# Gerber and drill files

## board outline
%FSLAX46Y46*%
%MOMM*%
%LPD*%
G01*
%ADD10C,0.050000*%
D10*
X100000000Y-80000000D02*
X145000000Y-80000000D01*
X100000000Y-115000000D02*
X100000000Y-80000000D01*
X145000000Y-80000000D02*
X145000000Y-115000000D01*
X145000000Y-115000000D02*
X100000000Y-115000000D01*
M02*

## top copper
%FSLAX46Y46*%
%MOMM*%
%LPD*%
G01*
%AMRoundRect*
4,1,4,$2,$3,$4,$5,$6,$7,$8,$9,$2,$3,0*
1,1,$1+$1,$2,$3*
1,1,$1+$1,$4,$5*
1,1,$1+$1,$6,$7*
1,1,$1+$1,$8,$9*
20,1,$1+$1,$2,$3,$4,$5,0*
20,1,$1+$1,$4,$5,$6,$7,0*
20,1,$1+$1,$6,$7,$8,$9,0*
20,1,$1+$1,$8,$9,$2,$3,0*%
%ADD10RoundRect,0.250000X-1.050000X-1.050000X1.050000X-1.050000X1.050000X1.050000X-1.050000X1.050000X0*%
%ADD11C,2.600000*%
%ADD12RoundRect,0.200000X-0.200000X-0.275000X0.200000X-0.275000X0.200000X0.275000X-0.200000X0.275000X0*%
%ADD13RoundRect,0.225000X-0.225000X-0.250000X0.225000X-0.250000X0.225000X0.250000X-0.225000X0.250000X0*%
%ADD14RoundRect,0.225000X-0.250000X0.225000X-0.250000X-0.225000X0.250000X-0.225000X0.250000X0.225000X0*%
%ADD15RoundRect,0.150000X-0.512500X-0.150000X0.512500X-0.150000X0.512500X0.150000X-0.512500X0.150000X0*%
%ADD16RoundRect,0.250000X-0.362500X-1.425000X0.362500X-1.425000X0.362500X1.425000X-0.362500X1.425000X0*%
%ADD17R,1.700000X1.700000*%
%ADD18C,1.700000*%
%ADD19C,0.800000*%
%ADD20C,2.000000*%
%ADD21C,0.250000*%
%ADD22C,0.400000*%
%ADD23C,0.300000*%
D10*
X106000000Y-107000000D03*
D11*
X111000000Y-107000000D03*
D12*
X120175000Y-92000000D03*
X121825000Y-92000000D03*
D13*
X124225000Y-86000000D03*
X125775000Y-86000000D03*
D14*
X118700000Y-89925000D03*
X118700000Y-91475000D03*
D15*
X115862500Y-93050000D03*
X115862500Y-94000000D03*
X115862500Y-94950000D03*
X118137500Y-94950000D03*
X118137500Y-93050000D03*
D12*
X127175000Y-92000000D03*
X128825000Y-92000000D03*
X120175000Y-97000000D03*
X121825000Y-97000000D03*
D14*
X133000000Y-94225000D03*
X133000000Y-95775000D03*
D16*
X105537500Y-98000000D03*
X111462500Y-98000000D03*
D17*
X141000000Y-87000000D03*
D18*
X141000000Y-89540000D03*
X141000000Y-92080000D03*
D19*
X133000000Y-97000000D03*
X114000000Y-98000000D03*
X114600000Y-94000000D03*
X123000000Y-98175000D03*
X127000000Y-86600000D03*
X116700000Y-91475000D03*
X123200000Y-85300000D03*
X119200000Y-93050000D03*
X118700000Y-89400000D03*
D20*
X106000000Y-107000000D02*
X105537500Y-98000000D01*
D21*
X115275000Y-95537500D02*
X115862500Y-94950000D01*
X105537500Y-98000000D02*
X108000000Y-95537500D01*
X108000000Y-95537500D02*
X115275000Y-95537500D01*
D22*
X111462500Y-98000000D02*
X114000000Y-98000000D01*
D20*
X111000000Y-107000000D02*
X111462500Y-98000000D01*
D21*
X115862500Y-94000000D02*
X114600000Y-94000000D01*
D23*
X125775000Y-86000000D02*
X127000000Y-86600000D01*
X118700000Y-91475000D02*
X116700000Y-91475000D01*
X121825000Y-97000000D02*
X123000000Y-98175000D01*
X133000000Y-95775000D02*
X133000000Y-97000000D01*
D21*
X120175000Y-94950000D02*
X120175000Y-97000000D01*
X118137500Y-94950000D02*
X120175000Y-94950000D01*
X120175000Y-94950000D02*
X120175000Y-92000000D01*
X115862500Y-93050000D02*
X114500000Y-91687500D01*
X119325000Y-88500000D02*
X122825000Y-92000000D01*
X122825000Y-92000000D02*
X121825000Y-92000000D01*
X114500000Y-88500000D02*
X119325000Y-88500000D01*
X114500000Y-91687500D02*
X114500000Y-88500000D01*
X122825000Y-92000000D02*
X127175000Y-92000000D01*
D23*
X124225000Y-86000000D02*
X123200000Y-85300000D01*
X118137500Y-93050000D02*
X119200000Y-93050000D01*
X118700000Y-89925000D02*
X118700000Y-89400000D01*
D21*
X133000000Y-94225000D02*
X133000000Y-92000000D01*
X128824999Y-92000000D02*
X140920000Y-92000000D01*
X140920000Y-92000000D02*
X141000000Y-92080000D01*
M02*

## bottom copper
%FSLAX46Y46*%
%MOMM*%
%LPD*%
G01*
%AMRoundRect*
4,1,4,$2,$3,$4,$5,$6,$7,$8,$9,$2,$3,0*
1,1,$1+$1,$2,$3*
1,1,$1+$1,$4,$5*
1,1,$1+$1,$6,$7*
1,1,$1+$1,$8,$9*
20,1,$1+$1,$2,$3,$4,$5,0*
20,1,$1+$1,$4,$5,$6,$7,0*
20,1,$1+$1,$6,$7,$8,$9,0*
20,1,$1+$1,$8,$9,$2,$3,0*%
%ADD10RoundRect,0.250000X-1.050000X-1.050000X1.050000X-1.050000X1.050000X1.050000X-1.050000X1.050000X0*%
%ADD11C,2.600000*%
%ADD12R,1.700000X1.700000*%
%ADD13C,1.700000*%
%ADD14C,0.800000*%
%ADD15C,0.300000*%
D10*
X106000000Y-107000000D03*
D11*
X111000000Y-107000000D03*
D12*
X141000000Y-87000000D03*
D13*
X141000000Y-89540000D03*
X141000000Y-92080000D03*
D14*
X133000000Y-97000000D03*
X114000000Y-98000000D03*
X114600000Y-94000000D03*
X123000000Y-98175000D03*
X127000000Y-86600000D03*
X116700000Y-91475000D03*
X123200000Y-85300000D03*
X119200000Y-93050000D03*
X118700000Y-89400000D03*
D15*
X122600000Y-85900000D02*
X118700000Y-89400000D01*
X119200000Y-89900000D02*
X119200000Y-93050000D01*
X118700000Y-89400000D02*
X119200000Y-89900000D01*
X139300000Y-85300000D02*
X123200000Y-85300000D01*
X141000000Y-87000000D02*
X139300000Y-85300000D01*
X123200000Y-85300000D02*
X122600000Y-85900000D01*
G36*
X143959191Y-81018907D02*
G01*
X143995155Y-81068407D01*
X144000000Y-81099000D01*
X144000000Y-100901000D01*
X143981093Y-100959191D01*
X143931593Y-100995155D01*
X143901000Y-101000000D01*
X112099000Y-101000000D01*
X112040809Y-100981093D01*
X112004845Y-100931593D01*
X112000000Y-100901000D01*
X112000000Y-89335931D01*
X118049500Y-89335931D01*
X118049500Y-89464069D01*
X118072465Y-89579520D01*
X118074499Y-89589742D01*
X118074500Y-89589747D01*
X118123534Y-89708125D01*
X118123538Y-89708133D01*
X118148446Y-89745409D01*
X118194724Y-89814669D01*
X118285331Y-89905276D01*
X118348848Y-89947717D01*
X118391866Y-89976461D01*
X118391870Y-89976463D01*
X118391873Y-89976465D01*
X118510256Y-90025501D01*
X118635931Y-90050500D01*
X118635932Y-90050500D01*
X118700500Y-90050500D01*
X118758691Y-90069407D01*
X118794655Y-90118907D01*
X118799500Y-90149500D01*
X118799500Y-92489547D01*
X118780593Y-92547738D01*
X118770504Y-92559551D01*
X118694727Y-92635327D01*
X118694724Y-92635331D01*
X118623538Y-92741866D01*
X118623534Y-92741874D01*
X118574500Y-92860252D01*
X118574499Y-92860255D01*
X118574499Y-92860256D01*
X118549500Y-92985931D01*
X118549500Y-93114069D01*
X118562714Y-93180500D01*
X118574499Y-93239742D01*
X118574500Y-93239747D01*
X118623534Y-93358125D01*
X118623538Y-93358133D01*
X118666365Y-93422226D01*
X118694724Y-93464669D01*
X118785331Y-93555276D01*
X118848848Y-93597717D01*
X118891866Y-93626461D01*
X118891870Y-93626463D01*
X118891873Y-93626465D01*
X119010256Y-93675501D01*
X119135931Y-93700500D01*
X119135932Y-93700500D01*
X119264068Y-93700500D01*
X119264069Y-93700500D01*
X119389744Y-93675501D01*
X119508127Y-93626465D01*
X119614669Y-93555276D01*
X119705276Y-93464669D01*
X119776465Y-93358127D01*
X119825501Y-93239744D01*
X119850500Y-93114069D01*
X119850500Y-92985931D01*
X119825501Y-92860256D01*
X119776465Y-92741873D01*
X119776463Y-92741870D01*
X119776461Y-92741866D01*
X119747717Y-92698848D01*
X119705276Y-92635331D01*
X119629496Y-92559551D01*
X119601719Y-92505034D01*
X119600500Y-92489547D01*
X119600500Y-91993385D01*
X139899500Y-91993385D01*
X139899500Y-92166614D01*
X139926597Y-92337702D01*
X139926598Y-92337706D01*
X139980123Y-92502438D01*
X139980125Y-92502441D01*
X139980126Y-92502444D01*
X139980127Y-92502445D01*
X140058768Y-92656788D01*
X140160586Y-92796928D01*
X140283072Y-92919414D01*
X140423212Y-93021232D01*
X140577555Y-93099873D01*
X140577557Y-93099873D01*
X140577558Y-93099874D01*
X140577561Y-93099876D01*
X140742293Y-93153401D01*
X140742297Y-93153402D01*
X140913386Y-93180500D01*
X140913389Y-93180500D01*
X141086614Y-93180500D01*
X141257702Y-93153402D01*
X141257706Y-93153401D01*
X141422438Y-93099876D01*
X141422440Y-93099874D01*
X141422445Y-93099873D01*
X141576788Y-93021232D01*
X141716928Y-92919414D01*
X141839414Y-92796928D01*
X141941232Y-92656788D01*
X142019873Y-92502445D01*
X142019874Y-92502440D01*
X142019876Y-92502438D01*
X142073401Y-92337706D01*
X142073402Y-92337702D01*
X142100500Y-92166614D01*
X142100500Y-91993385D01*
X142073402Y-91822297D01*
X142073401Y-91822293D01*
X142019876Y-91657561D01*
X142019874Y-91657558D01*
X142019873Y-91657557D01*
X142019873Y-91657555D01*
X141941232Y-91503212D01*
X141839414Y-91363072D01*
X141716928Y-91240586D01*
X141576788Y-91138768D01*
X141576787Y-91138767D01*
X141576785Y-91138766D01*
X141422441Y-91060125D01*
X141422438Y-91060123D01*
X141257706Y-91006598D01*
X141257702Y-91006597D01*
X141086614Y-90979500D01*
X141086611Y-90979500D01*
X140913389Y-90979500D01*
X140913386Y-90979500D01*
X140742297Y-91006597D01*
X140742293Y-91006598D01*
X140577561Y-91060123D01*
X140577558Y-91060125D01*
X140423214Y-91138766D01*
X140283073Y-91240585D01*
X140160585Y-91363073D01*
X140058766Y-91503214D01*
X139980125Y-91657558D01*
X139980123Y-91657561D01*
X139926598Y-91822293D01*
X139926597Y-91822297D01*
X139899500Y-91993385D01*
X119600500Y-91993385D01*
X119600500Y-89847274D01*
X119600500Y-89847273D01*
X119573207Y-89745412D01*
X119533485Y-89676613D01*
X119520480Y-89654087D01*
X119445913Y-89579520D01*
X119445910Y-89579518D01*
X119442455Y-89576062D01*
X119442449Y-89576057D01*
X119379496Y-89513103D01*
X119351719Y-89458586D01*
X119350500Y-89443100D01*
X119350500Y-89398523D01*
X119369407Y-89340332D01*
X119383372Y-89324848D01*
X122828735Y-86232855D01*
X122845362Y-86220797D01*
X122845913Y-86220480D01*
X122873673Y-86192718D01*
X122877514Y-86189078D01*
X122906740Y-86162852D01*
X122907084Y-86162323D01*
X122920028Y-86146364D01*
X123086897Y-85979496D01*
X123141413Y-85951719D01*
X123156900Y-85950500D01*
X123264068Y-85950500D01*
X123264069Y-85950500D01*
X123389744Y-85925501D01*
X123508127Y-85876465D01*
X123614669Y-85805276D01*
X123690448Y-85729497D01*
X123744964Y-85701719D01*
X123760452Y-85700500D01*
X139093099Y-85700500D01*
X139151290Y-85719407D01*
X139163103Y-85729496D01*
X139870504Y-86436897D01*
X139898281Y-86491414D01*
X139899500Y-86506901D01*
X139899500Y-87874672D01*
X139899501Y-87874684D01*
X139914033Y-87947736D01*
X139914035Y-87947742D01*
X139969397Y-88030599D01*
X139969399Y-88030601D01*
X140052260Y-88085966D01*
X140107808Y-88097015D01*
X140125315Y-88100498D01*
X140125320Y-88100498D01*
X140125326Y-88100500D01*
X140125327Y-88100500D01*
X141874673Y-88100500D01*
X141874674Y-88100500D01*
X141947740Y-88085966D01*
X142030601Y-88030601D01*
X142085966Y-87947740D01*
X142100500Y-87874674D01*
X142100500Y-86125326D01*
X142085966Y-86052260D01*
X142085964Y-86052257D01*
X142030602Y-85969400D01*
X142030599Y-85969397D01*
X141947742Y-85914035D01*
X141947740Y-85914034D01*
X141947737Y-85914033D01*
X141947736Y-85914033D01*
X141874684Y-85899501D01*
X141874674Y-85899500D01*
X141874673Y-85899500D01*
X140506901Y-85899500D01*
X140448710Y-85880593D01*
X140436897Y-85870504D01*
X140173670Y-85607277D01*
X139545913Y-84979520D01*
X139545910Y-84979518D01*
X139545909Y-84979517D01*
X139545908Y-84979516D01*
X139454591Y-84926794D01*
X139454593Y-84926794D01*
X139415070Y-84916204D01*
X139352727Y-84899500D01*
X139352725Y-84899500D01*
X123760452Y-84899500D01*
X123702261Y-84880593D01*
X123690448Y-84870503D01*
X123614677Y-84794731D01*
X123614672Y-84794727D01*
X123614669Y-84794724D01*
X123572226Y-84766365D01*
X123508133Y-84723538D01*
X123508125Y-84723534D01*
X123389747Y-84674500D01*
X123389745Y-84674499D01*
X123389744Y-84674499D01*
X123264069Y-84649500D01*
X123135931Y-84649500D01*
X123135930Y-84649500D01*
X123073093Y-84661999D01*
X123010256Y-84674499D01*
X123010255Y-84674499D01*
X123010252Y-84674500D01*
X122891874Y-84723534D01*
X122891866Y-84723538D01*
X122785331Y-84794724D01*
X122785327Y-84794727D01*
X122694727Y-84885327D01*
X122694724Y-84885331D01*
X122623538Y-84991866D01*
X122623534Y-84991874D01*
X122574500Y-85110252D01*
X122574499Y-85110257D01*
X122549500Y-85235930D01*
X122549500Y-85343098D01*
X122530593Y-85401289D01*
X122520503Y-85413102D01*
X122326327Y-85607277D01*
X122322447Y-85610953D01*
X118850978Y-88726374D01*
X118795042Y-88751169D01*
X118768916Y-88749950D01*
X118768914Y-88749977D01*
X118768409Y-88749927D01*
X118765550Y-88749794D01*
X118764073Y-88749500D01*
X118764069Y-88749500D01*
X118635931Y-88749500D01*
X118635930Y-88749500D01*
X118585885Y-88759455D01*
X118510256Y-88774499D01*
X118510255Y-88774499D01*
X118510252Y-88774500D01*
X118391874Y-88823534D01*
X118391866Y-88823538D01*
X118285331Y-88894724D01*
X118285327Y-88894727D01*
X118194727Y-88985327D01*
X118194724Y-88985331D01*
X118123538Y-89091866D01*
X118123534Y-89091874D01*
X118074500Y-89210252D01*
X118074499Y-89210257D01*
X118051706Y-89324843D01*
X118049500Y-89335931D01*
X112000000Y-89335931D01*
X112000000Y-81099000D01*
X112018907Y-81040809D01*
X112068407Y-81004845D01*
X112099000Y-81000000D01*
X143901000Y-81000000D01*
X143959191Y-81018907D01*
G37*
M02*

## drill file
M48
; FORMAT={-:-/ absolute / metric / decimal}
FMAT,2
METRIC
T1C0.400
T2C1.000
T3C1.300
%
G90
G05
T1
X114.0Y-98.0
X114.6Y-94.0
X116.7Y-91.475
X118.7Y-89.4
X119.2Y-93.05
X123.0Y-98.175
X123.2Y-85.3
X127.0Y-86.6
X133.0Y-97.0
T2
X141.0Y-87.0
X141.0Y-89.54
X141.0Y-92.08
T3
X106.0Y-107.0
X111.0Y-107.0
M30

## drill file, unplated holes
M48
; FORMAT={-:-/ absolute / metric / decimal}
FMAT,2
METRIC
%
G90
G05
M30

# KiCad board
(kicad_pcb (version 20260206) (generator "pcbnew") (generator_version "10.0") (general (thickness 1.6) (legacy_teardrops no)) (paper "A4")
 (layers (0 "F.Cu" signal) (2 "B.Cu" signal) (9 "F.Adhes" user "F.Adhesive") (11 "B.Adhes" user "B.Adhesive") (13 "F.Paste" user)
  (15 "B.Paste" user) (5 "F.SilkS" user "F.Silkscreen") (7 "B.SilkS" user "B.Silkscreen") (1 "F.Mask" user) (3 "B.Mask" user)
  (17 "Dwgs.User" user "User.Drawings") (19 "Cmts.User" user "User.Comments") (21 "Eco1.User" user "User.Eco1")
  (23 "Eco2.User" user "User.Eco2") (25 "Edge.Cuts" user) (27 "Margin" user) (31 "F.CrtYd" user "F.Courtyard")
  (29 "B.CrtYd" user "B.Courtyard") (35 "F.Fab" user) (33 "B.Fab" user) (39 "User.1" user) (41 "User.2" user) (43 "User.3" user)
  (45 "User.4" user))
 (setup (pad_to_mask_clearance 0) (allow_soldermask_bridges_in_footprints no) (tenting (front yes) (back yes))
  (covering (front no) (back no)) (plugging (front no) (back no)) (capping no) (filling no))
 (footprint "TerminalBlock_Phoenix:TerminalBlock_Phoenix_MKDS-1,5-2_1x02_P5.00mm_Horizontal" (layer "F.Cu") (at 106 107)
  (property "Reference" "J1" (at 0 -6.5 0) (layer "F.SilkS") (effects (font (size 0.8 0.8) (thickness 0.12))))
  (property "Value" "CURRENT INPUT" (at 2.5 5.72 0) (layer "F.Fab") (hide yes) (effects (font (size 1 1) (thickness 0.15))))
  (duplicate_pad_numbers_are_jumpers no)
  (pad "1" thru_hole roundrect (at 0 0) (size 2.6 2.6) (drill 1.3) (layers "*.Cu" "*.Mask") (remove_unused_layers no)
   (roundrect_rratio 0.096154) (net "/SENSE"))
  (pad "2" thru_hole circle (at 5 0) (size 2.6 2.6) (drill 1.3) (layers "*.Cu" "*.Mask") (remove_unused_layers no) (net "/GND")))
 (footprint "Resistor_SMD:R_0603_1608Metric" (layer "F.Cu") (at 121 92)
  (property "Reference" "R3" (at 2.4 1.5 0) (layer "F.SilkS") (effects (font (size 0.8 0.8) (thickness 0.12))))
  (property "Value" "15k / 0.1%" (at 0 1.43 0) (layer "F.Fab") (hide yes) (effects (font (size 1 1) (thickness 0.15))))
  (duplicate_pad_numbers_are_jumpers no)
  (pad "1" smd roundrect (at -0.825 0) (size 0.8 0.95) (layers "F.Cu" "F.Mask" "F.Paste") (roundrect_rratio 0.25) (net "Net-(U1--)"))
  (pad "2" smd roundrect (at 0.825 0) (size 0.8 0.95) (layers "F.Cu" "F.Mask" "F.Paste") (roundrect_rratio 0.25) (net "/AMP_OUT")))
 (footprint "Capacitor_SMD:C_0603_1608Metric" (layer "F.Cu") (at 125 86)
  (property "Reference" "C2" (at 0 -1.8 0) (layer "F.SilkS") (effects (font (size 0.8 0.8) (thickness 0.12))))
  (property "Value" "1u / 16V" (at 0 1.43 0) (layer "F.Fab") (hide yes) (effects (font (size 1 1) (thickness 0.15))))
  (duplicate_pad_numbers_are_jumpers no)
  (pad "1" smd roundrect (at -0.775 0) (size 0.9 0.95) (layers "F.Cu" "F.Mask" "F.Paste") (roundrect_rratio 0.25) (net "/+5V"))
  (pad "2" smd roundrect (at 0.775 0) (size 0.9 0.95) (layers "F.Cu" "F.Mask" "F.Paste") (roundrect_rratio 0.25) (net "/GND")))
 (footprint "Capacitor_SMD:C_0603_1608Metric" (layer "F.Cu") (at 118.7 90.7 -90)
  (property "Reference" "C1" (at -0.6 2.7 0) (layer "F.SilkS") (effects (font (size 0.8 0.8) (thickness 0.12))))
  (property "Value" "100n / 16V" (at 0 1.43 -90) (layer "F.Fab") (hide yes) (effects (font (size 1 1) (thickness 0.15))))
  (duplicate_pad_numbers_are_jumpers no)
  (pad "1" smd roundrect (at -0.775 0 270) (size 0.9 0.95) (layers "F.Cu" "F.Mask" "F.Paste") (roundrect_rratio 0.25) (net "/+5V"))
  (pad "2" smd roundrect (at 0.775 0 270) (size 0.9 0.95) (layers "F.Cu" "F.Mask" "F.Paste") (roundrect_rratio 0.25) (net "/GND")))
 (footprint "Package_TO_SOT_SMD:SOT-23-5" (layer "F.Cu") (at 117 94)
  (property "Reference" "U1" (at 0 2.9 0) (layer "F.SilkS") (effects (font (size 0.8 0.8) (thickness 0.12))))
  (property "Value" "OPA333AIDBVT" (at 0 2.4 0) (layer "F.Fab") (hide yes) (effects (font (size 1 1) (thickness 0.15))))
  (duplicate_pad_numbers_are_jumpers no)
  (pad "1" smd roundrect (at -1.1375 -0.95) (size 1.325 0.6) (layers "F.Cu" "F.Mask" "F.Paste") (roundrect_rratio 0.25) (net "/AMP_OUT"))
  (pad "2" smd roundrect (at -1.1375 0) (size 1.325 0.6) (layers "F.Cu" "F.Mask" "F.Paste") (roundrect_rratio 0.25) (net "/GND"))
  (pad "3" smd roundrect (at -1.1375 0.95) (size 1.325 0.6) (layers "F.Cu" "F.Mask" "F.Paste") (roundrect_rratio 0.25) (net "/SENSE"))
  (pad "4" smd roundrect (at 1.1375 0.95) (size 1.325 0.6) (layers "F.Cu" "F.Mask" "F.Paste") (roundrect_rratio 0.25) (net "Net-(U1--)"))
  (pad "5" smd roundrect (at 1.1375 -0.95) (size 1.325 0.6) (layers "F.Cu" "F.Mask" "F.Paste") (roundrect_rratio 0.25) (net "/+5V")))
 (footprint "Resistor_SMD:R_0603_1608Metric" (layer "F.Cu") (at 128 92)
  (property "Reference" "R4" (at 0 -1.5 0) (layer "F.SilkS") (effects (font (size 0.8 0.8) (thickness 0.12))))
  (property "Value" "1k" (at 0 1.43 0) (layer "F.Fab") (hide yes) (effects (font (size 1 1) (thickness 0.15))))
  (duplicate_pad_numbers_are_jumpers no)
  (pad "1" smd roundrect (at -0.825 0) (size 0.8 0.95) (layers "F.Cu" "F.Mask" "F.Paste") (roundrect_rratio 0.25) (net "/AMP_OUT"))
  (pad "2" smd roundrect (at 0.825 0) (size 0.8 0.95) (layers "F.Cu" "F.Mask" "F.Paste") (roundrect_rratio 0.25) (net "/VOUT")))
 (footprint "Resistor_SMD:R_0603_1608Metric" (layer "F.Cu") (at 121 97)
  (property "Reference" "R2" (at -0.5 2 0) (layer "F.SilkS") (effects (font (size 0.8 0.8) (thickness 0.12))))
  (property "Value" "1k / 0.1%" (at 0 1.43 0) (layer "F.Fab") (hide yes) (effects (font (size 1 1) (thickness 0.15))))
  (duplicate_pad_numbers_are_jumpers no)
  (pad "1" smd roundrect (at -0.825 0) (size 0.8 0.95) (layers "F.Cu" "F.Mask" "F.Paste") (roundrect_rratio 0.25) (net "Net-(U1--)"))
  (pad "2" smd roundrect (at 0.825 0) (size 0.8 0.95) (layers "F.Cu" "F.Mask" "F.Paste") (roundrect_rratio 0.25) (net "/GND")))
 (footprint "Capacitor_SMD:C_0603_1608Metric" (layer "F.Cu") (at 133 95 -90)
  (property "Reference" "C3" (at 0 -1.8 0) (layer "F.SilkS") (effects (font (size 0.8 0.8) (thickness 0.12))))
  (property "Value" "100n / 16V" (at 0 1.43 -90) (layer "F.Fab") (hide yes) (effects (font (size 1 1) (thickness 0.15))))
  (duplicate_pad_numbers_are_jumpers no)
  (pad "1" smd roundrect (at -0.775 0 270) (size 0.9 0.95) (layers "F.Cu" "F.Mask" "F.Paste") (roundrect_rratio 0.25) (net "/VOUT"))
  (pad "2" smd roundrect (at 0.775 0 270) (size 0.9 0.95) (layers "F.Cu" "F.Mask" "F.Paste") (roundrect_rratio 0.25) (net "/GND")))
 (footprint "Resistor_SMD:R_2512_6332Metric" (layer "F.Cu") (at 108.5 98)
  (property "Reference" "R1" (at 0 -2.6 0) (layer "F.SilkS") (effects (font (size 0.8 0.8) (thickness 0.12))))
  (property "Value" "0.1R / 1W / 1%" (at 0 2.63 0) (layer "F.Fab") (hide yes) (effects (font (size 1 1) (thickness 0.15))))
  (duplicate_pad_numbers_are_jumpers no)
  (pad "1" smd roundrect (at -2.9625 0) (size 1.225 3.35) (layers "F.Cu" "F.Mask" "F.Paste") (roundrect_rratio 0.204082) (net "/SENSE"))
  (pad "2" smd roundrect (at 2.9625 0) (size 1.225 3.35) (layers "F.Cu" "F.Mask" "F.Paste") (roundrect_rratio 0.204082) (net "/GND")))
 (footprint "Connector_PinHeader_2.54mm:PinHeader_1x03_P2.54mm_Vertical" (layer "F.Cu") (at 141 87)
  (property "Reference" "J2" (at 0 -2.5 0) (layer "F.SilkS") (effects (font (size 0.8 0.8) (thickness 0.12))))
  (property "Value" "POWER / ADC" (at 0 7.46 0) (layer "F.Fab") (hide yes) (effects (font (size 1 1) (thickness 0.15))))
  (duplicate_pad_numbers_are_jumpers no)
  (pad "1" thru_hole rect (at 0 0) (size 1.7 1.7) (drill 1) (layers "*.Cu" "*.Mask") (remove_unused_layers no) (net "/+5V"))
  (pad "2" thru_hole circle (at 0 2.54) (size 1.7 1.7) (drill 1) (layers "*.Cu" "*.Mask") (remove_unused_layers no) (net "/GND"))
  (pad "3" thru_hole circle (at 0 5.08) (size 1.7 1.7) (drill 1) (layers "*.Cu" "*.Mask") (remove_unused_layers no) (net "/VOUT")))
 (gr_line (start 100 80) (end 145 80) (stroke (width 0.05) (type default)) (layer "Edge.Cuts"))
 (gr_line (start 100 115) (end 100 80) (stroke (width 0.05) (type default)) (layer "Edge.Cuts"))
 (gr_line (start 145 80) (end 145 115) (stroke (width 0.05) (type default)) (layer "Edge.Cuts"))
 (gr_line (start 145 115) (end 100 115) (stroke (width 0.05) (type default)) (layer "Edge.Cuts"))
 (segment (start 106 107) (end 105.5375 98) (width 2) (layer "F.Cu") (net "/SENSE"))
 (segment (start 115.275 95.5375) (end 115.8625 94.95) (width 0.25) (layer "F.Cu") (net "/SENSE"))
 (segment (start 105.5375 98) (end 108 95.5375) (width 0.25) (layer "F.Cu") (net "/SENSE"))
 (segment (start 108 95.5375) (end 115.275 95.5375) (width 0.25) (layer "F.Cu") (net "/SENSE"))
 (segment (start 111.4625 98) (end 114 98) (width 0.4) (layer "F.Cu") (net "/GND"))
 (segment (start 111 107) (end 111.4625 98) (width 2) (layer "F.Cu") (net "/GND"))
 (segment (start 115.8625 94) (end 114.6 94) (width 0.25) (layer "F.Cu") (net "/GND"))
 (segment (start 125.775 86) (end 127 86.6) (width 0.3) (layer "F.Cu") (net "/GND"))
 (segment (start 118.7 91.475) (end 116.7 91.475) (width 0.3) (layer "F.Cu") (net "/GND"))
 (segment (start 121.825 97) (end 123 98.175) (width 0.3) (layer "F.Cu") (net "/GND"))
 (segment (start 133 95.775) (end 133 97) (width 0.3) (layer "F.Cu") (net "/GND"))
 (via (at 133 97) (size 0.8) (drill 0.4) (layers "F.Cu" "B.Cu") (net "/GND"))
 (via (at 114 98) (size 0.8) (drill 0.4) (layers "F.Cu" "B.Cu") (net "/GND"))
 (via (at 114.6 94) (size 0.8) (drill 0.4) (layers "F.Cu" "B.Cu") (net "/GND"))
 (via (at 123 98.175) (size 0.8) (drill 0.4) (layers "F.Cu" "B.Cu") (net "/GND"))
 (via (at 127 86.6) (size 0.8) (drill 0.4) (layers "F.Cu" "B.Cu") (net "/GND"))
 (via (at 116.7 91.475) (size 0.8) (drill 0.4) (layers "F.Cu" "B.Cu") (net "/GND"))
 (segment (start 120.175 94.95) (end 120.175 97) (width 0.25) (layer "F.Cu") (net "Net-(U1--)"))
 (segment (start 118.1375 94.95) (end 120.175 94.95) (width 0.25) (layer "F.Cu") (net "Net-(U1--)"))
 (segment (start 120.175 94.95) (end 120.175 92) (width 0.25) (layer "F.Cu") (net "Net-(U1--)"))
 (segment (start 115.8625 93.05) (end 114.5 91.6875) (width 0.25) (layer "F.Cu") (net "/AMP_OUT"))
 (segment (start 119.325 88.5) (end 122.825 92) (width 0.25) (layer "F.Cu") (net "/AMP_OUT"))
 (segment (start 122.825 92) (end 121.825 92) (width 0.25) (layer "F.Cu") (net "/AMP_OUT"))
 (segment (start 114.5 88.5) (end 119.325 88.5) (width 0.25) (layer "F.Cu") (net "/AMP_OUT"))
 (segment (start 114.5 91.6875) (end 114.5 88.5) (width 0.25) (layer "F.Cu") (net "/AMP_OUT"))
 (segment (start 122.825 92) (end 127.175 92) (width 0.25) (layer "F.Cu") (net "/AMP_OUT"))
 (segment (start 124.225 86) (end 123.2 85.3) (width 0.3) (layer "F.Cu") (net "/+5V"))
 (segment (start 118.1375 93.05) (end 119.2 93.05) (width 0.3) (layer "F.Cu") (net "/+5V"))
 (segment (start 118.7 89.925) (end 118.7 89.4) (width 0.3) (layer "F.Cu") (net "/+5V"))
 (via (at 123.2 85.3) (size 0.8) (drill 0.4) (layers "F.Cu" "B.Cu") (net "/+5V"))
 (via (at 119.2 93.05) (size 0.8) (drill 0.4) (layers "F.Cu" "B.Cu") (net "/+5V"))
 (via (at 118.7 89.4) (size 0.8) (drill 0.4) (layers "F.Cu" "B.Cu") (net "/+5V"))
 (segment (start 122.6 85.9) (end 118.7 89.4) (width 0.3) (layer "B.Cu") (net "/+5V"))
 (segment (start 119.2 89.9) (end 119.2 93.05) (width 0.3) (layer "B.Cu") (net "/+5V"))
 (segment (start 118.7 89.4) (end 119.2 89.9) (width 0.3) (layer "B.Cu") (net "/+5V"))
 (segment (start 139.3 85.3) (end 123.2 85.3) (width 0.3) (layer "B.Cu") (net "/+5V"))
 (segment (start 141 87) (end 139.3 85.3) (width 0.3) (layer "B.Cu") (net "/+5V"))
 (segment (start 123.2 85.3) (end 122.6 85.9) (width 0.3) (layer "B.Cu") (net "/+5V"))
 (segment (start 133 94.225) (end 133 92) (width 0.25) (layer "F.Cu") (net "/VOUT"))
 (segment (start 128.824999 92) (end 140.92 92) (width 0.25) (layer "F.Cu") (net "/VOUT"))
 (segment (start 140.92 92) (end 141 92.08) (width 0.25) (layer "F.Cu") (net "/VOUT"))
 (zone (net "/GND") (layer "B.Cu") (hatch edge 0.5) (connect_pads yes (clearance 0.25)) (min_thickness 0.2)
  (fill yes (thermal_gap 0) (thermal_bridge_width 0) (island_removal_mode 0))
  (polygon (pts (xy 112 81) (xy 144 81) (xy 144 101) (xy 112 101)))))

